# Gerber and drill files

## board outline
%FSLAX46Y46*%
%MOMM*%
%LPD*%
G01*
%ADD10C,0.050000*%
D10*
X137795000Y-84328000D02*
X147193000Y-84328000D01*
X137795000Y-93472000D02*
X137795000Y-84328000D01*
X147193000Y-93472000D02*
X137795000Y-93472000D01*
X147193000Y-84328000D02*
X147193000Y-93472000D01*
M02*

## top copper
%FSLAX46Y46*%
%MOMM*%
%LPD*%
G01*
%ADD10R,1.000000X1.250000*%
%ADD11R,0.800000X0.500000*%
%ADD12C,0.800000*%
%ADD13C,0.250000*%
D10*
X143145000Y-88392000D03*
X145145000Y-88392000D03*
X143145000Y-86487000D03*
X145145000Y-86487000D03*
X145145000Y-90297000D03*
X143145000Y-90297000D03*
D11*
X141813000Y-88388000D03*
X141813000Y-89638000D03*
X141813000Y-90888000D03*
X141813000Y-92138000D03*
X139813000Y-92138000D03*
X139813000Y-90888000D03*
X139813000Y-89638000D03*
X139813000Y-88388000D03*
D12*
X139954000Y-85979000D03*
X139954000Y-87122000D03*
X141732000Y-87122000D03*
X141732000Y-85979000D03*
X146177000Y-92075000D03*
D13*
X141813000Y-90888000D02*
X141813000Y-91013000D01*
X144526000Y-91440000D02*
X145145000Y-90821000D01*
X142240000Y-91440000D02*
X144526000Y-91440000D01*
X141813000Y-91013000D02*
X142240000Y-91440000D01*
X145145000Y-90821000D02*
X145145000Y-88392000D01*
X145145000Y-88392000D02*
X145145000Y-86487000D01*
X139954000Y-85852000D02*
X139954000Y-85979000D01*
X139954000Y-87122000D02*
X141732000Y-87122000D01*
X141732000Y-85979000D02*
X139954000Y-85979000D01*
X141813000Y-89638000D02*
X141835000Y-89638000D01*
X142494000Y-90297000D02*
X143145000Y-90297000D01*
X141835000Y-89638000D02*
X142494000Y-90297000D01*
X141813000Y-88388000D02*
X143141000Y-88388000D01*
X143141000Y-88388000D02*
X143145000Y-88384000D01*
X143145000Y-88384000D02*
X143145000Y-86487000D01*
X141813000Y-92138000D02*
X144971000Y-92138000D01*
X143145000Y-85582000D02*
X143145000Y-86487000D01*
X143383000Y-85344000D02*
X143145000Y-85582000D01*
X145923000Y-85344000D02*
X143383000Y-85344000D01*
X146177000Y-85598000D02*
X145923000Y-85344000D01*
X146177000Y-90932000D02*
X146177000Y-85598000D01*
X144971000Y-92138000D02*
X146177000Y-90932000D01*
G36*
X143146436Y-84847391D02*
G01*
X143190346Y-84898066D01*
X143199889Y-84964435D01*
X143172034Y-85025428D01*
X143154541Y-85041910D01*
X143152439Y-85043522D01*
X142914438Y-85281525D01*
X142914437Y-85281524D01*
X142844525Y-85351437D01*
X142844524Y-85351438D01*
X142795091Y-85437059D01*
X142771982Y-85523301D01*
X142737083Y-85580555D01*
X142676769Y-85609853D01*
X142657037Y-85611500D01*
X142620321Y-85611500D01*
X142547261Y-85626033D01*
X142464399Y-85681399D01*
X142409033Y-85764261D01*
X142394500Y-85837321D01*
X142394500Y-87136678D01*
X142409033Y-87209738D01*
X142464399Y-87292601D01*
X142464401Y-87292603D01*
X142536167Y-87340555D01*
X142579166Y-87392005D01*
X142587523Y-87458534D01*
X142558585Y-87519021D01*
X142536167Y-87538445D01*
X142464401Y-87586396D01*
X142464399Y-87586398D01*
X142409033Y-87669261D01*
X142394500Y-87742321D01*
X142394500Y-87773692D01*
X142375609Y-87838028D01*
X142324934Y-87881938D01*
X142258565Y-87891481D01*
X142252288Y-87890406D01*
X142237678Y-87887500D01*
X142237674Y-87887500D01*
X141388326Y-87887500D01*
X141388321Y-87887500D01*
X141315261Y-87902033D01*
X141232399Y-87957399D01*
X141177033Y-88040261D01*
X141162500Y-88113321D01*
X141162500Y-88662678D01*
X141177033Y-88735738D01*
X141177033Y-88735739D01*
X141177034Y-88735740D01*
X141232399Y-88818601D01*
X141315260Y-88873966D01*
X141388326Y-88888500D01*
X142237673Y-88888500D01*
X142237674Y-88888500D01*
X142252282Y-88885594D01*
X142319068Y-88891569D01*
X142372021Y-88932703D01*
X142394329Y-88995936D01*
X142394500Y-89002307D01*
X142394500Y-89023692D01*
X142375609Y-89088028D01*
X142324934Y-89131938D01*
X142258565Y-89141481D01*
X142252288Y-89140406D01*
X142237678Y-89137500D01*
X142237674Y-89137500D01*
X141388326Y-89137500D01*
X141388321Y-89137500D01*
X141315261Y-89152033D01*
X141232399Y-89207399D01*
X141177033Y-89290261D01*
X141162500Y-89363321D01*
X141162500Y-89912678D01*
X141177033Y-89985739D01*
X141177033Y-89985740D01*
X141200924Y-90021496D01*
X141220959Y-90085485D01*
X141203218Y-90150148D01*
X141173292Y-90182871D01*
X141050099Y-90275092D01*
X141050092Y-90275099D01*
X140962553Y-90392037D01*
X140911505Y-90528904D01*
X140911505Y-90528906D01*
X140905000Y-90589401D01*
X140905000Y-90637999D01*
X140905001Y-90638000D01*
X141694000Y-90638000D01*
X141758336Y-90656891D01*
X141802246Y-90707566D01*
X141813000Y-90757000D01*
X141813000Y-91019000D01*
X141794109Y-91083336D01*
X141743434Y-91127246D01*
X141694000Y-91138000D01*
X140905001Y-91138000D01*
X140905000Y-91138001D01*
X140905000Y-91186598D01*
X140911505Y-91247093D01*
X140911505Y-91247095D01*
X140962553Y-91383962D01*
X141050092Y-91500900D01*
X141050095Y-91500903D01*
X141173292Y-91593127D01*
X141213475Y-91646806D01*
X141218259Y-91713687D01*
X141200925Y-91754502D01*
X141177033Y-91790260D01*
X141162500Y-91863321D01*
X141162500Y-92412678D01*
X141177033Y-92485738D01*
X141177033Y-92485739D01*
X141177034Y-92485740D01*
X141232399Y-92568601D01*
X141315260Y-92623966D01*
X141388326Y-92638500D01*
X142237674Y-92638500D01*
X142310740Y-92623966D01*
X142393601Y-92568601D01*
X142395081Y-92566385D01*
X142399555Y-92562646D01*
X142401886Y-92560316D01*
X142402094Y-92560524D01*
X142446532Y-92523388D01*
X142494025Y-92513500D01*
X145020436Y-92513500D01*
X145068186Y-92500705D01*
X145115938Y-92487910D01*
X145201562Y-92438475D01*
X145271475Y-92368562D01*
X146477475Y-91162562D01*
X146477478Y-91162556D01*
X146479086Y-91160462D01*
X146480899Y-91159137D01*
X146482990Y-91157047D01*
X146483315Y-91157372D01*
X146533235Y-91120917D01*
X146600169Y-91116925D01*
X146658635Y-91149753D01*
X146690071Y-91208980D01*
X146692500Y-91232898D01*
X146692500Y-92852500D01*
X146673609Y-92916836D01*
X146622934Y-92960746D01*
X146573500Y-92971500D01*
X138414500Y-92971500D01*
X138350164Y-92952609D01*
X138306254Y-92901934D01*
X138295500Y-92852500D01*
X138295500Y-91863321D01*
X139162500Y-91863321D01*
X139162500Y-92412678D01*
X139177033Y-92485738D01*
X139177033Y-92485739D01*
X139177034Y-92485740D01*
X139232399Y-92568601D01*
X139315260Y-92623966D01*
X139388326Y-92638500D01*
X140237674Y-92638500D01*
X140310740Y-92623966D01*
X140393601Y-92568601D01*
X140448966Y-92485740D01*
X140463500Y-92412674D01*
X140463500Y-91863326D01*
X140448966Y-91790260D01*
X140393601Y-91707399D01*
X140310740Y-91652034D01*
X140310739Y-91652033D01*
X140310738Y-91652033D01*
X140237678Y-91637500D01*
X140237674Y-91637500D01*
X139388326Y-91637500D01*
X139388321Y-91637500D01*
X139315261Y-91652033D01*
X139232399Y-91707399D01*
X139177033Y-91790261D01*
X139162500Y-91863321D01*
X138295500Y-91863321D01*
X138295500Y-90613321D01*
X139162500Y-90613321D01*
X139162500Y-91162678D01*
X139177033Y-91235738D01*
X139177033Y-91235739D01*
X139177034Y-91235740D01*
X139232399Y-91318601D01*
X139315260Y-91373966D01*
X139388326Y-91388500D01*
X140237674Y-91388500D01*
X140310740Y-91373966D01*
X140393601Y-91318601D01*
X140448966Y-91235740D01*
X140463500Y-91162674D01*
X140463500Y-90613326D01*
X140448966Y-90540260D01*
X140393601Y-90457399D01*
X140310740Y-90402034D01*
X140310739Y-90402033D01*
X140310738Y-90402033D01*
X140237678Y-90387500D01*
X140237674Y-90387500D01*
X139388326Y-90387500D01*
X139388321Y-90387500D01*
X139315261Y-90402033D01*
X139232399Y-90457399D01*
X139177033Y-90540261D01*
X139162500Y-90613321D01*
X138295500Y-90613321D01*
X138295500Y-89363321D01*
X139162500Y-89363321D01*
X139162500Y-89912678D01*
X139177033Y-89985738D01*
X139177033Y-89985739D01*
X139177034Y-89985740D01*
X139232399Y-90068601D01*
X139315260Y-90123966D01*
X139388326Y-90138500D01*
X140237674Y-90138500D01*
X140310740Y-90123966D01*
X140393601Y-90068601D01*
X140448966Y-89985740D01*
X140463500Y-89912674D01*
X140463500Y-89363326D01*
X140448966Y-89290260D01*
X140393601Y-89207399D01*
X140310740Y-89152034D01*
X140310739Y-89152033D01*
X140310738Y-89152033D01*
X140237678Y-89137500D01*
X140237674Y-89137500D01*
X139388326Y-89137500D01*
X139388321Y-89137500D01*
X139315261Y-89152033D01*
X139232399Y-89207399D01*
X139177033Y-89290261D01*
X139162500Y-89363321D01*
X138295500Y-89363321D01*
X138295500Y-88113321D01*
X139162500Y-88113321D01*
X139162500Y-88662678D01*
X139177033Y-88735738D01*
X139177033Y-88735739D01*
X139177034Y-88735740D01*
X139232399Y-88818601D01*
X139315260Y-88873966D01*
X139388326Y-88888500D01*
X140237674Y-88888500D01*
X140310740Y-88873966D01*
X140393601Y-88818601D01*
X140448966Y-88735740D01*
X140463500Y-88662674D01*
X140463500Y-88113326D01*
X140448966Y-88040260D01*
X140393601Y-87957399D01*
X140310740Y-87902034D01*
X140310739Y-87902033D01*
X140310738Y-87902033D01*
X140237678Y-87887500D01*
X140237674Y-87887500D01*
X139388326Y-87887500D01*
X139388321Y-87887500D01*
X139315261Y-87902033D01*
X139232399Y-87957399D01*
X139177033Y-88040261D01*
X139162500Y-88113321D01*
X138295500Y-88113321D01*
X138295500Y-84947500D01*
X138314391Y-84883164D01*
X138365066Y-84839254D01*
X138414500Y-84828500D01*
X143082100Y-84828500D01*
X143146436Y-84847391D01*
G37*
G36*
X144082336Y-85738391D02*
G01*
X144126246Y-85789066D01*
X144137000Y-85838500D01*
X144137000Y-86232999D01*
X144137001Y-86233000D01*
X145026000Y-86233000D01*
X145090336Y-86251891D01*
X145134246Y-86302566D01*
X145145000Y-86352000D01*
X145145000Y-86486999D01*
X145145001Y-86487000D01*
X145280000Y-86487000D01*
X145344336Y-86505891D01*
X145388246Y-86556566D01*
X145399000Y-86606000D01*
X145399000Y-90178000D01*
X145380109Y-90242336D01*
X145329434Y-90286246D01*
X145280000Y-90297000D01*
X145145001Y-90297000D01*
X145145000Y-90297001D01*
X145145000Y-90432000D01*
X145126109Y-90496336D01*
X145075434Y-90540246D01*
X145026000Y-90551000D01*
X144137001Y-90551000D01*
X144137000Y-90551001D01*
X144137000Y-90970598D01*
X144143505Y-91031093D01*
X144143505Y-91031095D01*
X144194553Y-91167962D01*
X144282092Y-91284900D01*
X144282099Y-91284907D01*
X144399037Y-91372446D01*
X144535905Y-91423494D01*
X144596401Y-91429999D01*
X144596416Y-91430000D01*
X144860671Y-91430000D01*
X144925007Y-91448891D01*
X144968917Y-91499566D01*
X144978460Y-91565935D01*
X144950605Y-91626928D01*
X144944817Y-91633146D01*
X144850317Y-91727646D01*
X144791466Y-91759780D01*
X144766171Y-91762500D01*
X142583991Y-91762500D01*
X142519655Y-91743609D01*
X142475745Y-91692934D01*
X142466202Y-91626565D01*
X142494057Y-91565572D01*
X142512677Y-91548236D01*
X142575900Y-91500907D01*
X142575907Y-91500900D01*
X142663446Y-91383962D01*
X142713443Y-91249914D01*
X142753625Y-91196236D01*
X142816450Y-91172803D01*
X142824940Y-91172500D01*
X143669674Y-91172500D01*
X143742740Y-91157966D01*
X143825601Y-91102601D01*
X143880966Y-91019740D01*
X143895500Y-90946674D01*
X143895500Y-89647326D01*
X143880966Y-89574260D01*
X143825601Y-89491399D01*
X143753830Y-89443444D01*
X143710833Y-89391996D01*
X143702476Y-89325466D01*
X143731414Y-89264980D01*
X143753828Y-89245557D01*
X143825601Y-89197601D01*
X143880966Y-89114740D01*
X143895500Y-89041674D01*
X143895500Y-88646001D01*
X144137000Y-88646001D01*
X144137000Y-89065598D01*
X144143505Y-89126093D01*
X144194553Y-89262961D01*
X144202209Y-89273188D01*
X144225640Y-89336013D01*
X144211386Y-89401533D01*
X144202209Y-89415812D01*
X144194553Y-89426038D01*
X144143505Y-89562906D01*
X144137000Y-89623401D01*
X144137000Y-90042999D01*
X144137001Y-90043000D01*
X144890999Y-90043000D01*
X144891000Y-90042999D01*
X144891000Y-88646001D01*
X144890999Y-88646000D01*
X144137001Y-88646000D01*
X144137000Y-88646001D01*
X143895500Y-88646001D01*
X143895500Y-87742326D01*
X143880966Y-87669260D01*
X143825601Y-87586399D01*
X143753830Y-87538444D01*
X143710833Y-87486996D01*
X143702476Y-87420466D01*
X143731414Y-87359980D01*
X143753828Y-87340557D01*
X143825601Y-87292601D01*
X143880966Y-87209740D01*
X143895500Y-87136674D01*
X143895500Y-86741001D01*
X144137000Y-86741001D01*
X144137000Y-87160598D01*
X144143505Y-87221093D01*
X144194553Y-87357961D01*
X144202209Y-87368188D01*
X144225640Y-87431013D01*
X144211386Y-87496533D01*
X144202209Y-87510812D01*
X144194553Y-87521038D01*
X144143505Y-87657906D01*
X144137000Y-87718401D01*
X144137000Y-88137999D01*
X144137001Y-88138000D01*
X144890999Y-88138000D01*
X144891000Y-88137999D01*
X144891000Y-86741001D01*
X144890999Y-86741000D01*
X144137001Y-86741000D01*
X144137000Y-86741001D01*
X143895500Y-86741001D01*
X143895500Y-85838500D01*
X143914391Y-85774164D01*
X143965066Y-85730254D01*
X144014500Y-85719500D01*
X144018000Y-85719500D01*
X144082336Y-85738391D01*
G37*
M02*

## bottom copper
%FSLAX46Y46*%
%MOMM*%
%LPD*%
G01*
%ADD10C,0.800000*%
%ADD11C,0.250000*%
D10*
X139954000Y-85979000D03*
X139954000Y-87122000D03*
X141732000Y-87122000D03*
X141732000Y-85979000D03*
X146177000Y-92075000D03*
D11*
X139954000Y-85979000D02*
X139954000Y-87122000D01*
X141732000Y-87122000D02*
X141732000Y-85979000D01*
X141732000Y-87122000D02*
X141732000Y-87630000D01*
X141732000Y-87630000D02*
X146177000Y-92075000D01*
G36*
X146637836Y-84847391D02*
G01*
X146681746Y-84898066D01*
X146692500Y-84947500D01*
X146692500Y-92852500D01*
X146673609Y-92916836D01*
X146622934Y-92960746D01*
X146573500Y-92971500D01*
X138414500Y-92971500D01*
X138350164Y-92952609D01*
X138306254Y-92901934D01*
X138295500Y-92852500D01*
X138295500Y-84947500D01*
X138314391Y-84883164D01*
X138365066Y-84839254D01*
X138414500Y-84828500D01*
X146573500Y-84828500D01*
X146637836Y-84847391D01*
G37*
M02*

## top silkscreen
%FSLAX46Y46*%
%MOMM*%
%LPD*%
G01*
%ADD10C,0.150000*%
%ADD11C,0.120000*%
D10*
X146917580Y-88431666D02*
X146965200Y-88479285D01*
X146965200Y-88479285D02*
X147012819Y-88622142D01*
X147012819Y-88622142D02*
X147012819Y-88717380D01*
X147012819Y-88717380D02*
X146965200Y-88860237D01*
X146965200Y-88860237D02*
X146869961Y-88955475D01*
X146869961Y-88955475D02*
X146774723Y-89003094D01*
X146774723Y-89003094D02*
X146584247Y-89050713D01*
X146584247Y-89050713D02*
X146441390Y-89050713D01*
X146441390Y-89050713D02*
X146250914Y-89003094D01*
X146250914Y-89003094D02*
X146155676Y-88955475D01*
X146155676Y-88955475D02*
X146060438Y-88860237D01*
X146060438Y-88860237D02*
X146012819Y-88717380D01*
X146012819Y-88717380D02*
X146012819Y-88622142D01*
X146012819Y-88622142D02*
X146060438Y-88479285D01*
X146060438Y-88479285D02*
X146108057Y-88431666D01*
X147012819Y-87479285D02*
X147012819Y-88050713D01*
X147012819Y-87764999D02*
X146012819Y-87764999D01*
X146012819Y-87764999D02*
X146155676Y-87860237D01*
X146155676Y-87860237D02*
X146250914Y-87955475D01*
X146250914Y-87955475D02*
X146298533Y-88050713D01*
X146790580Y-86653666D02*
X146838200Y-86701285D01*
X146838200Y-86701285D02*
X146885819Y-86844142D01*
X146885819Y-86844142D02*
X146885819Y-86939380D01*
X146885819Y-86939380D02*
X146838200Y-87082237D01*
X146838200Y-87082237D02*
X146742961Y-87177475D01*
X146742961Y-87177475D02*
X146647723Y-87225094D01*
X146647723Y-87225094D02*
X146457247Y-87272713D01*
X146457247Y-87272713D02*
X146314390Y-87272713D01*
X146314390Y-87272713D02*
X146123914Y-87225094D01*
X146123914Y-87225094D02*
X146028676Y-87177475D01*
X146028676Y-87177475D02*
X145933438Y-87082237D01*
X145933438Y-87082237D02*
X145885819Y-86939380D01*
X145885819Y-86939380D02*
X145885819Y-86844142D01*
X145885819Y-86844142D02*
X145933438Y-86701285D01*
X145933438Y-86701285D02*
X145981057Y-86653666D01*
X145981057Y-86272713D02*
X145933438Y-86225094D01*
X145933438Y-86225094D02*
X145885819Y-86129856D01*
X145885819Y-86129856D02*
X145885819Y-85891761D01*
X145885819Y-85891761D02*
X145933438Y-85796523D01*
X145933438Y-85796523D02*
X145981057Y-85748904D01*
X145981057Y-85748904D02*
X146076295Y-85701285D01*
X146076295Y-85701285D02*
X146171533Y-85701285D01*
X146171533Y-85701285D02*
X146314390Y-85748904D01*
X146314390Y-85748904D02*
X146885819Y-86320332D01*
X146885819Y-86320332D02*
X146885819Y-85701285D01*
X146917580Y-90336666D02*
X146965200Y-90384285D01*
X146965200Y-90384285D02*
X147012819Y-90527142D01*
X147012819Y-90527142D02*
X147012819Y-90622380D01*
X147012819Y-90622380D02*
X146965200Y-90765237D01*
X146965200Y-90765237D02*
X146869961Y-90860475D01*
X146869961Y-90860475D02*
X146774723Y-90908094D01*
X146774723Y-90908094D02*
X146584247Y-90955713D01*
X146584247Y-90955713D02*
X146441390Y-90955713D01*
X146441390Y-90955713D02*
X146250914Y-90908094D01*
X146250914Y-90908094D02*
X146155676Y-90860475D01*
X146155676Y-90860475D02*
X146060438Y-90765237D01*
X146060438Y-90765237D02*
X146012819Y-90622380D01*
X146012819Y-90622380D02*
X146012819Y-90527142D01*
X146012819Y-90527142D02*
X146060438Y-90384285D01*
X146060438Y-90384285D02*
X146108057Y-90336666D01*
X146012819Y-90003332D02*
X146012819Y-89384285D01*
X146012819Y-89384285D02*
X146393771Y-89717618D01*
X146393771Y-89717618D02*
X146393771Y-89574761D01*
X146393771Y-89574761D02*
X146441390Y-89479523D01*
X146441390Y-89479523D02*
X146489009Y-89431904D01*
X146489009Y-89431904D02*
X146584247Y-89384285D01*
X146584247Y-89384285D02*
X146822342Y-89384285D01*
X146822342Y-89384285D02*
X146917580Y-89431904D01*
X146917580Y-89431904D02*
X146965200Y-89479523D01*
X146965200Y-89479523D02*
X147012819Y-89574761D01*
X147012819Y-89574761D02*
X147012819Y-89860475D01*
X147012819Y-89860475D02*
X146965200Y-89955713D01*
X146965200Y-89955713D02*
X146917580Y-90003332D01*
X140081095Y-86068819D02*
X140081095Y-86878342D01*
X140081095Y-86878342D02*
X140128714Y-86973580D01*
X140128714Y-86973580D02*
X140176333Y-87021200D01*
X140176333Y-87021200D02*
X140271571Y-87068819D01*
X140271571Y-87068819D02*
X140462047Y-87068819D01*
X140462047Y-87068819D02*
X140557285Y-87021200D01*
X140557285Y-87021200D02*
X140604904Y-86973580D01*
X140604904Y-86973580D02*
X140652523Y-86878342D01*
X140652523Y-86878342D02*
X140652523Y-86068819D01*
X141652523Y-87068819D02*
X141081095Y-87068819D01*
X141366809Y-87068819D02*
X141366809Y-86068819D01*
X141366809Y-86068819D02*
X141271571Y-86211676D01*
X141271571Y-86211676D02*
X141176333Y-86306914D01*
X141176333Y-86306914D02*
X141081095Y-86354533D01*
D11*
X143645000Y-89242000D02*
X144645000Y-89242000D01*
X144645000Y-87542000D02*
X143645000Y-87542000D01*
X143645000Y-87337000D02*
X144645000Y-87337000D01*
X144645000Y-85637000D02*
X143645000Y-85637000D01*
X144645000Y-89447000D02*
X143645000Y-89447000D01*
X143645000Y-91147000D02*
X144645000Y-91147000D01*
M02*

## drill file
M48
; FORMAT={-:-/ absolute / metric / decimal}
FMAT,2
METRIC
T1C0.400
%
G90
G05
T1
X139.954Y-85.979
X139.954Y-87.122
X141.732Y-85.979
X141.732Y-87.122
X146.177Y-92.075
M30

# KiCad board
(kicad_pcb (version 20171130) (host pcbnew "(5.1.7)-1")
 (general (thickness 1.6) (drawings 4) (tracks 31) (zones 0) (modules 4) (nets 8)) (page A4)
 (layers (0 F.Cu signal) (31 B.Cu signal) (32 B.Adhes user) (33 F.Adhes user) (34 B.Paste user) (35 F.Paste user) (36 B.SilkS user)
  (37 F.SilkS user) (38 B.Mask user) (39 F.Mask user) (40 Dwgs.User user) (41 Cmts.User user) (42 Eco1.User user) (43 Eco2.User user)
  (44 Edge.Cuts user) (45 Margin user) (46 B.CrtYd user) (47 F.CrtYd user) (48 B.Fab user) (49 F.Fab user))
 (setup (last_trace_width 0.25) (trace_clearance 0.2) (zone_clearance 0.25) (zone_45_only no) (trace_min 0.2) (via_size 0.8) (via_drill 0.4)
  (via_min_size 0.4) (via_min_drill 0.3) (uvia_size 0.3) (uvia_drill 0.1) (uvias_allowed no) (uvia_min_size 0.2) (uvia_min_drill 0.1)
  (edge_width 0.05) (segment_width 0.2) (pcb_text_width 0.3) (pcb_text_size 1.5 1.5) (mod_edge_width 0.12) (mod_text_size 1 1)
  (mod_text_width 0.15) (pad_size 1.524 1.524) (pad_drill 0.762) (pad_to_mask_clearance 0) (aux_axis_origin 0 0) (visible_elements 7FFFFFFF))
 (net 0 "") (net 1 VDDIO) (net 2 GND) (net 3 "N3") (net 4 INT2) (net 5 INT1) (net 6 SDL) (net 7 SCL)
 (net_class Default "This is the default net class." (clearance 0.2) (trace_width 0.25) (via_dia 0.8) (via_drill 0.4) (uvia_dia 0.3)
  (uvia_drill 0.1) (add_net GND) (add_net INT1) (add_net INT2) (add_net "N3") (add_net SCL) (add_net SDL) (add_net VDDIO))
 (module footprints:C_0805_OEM (layer F.Cu) (at 144.145 88.392)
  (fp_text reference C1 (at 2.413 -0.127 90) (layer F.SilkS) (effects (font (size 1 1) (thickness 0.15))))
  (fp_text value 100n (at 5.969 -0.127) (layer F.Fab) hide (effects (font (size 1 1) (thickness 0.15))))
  (fp_line (start -0.5 0.85) (end 0.5 0.85) (layer F.SilkS) (width 0.12))
  (fp_line (start 0.5 -0.85) (end -0.5 -0.85) (layer F.SilkS) (width 0.12))
  (pad 1 smd rect (at -1 0) (size 1 1.25) (layers F.Cu F.Paste F.Mask) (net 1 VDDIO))
  (pad 2 smd rect (at 1 0) (size 1 1.25) (layers F.Cu F.Paste F.Mask) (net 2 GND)))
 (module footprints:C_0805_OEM (layer F.Cu) (at 144.145 86.487)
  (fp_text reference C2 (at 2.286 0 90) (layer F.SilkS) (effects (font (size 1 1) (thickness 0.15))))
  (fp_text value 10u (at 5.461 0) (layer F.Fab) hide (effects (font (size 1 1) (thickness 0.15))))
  (fp_line (start -0.5 0.85) (end 0.5 0.85) (layer F.SilkS) (width 0.12))
  (fp_line (start 0.5 -0.85) (end -0.5 -0.85) (layer F.SilkS) (width 0.12))
  (pad 1 smd rect (at -1 0) (size 1 1.25) (layers F.Cu F.Paste F.Mask) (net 1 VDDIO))
  (pad 2 smd rect (at 1 0) (size 1 1.25) (layers F.Cu F.Paste F.Mask) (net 2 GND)))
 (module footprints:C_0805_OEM (layer F.Cu) (at 144.145 90.297)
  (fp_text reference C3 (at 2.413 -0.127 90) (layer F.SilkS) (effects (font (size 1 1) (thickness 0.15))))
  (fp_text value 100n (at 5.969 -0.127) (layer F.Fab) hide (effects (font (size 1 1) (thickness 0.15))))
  (fp_line (start 0.5 -0.85) (end -0.5 -0.85) (layer F.SilkS) (width 0.12))
  (fp_line (start -0.5 0.85) (end 0.5 0.85) (layer F.SilkS) (width 0.12))
  (pad 2 smd rect (at 1 0) (size 1 1.25) (layers F.Cu F.Paste F.Mask) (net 2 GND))
  (pad 1 smd rect (at -1 0) (size 1 1.25) (layers F.Cu F.Paste F.Mask) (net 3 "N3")))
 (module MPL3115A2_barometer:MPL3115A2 (layer F.Cu) (at 140.813 90.263)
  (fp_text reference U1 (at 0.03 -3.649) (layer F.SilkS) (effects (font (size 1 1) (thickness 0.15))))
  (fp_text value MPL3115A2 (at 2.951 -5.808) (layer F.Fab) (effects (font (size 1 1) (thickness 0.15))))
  (pad 1 smd rect (at 1 -1.875) (size 0.8 0.5) (layers F.Cu F.Paste F.Mask) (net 1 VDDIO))
  (pad 2 smd rect (at 1 -0.625) (size 0.8 0.5) (layers F.Cu F.Paste F.Mask) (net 3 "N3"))
  (pad 3 smd rect (at 1 0.625) (size 0.8 0.5) (layers F.Cu F.Paste F.Mask) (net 2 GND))
  (pad 4 smd rect (at 1 1.875) (size 0.8 0.5) (layers F.Cu F.Paste F.Mask) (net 1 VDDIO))
  (pad 5 smd rect (at -1 1.875) (size 0.8 0.5) (layers F.Cu F.Paste F.Mask) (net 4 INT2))
  (pad 6 smd rect (at -1 0.625) (size 0.8 0.5) (layers F.Cu F.Paste F.Mask) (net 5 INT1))
  (pad 7 smd rect (at -1 -0.625) (size 0.8 0.5) (layers F.Cu F.Paste F.Mask) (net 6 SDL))
  (pad 8 smd rect (at -1 -1.875) (size 0.8 0.5) (layers F.Cu F.Paste F.Mask) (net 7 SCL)))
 (gr_line (start 137.795 84.328) (end 147.193 84.328) (angle 90) (layer Edge.Cuts) (width 0.05))
 (gr_line (start 137.795 93.472) (end 137.795 84.328) (angle 90) (layer Edge.Cuts) (width 0.05))
 (gr_line (start 147.193 93.472) (end 137.795 93.472) (angle 90) (layer Edge.Cuts) (width 0.05))
 (gr_line (start 147.193 84.328) (end 147.193 93.472) (angle 90) (layer Edge.Cuts) (width 0.05))
 (segment (start 141.813 90.888) (end 141.813 91.013) (width 0.25) (layer F.Cu) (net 2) (status C00000))
 (segment (start 144.526 91.44) (end 145.145 90.821) (width 0.25) (layer F.Cu) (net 2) (status 800000))
 (segment (start 142.24 91.44) (end 144.526 91.44) (width 0.25) (layer F.Cu) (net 2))
 (segment (start 141.813 91.013) (end 142.24 91.44) (width 0.25) (layer F.Cu) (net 2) (status 400000))
 (segment (start 145.145 90.821) (end 145.145 88.392) (width 0.25) (layer F.Cu) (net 2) (status C00000))
 (segment (start 145.145 88.392) (end 145.145 86.487) (width 0.25) (layer F.Cu) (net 2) (status C00000))
 (segment (start 139.954 85.852) (end 139.954 85.979) (width 0.25) (layer F.Cu) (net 2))
 (via (at 139.954 85.979) (size 0.8) (drill 0.4) (layers F.Cu B.Cu) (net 2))
 (segment (start 139.954 85.979) (end 139.954 87.122) (width 0.25) (layer B.Cu) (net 2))
 (via (at 139.954 87.122) (size 0.8) (drill 0.4) (layers F.Cu B.Cu) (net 2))
 (segment (start 139.954 87.122) (end 141.732 87.122) (width 0.25) (layer F.Cu) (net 2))
 (via (at 141.732 87.122) (size 0.8) (drill 0.4) (layers F.Cu B.Cu) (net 2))
 (segment (start 141.732 87.122) (end 141.732 85.979) (width 0.25) (layer B.Cu) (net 2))
 (via (at 141.732 85.979) (size 0.8) (drill 0.4) (layers F.Cu B.Cu) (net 2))
 (segment (start 141.732 85.979) (end 139.954 85.979) (width 0.25) (layer F.Cu) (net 2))
 (segment (start 141.732 87.122) (end 141.732 87.63) (width 0.25) (layer B.Cu) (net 2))
 (via (at 146.177 92.075) (size 0.8) (drill 0.4) (layers F.Cu B.Cu) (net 2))
 (segment (start 141.732 87.63) (end 146.177 92.075) (width 0.25) (layer B.Cu) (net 2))
 (segment (start 141.813 89.638) (end 141.835 89.638) (width 0.25) (layer F.Cu) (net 3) (status C00000))
 (segment (start 142.494 90.297) (end 143.145 90.297) (width 0.25) (layer F.Cu) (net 3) (status 800000))
 (segment (start 141.835 89.638) (end 142.494 90.297) (width 0.25) (layer F.Cu) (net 3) (status 400000))
 (segment (start 141.813 88.388) (end 143.141 88.388) (width 0.25) (layer F.Cu) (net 1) (status C00000))
 (segment (start 143.141 88.388) (end 143.145 88.384) (width 0.25) (layer F.Cu) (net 1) (status C00000))
 (segment (start 143.145 88.384) (end 143.145 86.487) (width 0.25) (layer F.Cu) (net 1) (status C00000))
 (segment (start 141.813 92.138) (end 144.971 92.138) (width 0.25) (layer F.Cu) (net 1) (status 400000))
 (segment (start 143.145 85.582) (end 143.145 86.487) (width 0.25) (layer F.Cu) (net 1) (status 800000))
 (segment (start 143.383 85.344) (end 143.145 85.582) (width 0.25) (layer F.Cu) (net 1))
 (segment (start 145.923 85.344) (end 143.383 85.344) (width 0.25) (layer F.Cu) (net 1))
 (segment (start 146.177 85.598) (end 145.923 85.344) (width 0.25) (layer F.Cu) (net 1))
 (segment (start 146.177 90.932) (end 146.177 85.598) (width 0.25) (layer F.Cu) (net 1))
 (segment (start 144.971 92.138) (end 146.177 90.932) (width 0.25) (layer F.Cu) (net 1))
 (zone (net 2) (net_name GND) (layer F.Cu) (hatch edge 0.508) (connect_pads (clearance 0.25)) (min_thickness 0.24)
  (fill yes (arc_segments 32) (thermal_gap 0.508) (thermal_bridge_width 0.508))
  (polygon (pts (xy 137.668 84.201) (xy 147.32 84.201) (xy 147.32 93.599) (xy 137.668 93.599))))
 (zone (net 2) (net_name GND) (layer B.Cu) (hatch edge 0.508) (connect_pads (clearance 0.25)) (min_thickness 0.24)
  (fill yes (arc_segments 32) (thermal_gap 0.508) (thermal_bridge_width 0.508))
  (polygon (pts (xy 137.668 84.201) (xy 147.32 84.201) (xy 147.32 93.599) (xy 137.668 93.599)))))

